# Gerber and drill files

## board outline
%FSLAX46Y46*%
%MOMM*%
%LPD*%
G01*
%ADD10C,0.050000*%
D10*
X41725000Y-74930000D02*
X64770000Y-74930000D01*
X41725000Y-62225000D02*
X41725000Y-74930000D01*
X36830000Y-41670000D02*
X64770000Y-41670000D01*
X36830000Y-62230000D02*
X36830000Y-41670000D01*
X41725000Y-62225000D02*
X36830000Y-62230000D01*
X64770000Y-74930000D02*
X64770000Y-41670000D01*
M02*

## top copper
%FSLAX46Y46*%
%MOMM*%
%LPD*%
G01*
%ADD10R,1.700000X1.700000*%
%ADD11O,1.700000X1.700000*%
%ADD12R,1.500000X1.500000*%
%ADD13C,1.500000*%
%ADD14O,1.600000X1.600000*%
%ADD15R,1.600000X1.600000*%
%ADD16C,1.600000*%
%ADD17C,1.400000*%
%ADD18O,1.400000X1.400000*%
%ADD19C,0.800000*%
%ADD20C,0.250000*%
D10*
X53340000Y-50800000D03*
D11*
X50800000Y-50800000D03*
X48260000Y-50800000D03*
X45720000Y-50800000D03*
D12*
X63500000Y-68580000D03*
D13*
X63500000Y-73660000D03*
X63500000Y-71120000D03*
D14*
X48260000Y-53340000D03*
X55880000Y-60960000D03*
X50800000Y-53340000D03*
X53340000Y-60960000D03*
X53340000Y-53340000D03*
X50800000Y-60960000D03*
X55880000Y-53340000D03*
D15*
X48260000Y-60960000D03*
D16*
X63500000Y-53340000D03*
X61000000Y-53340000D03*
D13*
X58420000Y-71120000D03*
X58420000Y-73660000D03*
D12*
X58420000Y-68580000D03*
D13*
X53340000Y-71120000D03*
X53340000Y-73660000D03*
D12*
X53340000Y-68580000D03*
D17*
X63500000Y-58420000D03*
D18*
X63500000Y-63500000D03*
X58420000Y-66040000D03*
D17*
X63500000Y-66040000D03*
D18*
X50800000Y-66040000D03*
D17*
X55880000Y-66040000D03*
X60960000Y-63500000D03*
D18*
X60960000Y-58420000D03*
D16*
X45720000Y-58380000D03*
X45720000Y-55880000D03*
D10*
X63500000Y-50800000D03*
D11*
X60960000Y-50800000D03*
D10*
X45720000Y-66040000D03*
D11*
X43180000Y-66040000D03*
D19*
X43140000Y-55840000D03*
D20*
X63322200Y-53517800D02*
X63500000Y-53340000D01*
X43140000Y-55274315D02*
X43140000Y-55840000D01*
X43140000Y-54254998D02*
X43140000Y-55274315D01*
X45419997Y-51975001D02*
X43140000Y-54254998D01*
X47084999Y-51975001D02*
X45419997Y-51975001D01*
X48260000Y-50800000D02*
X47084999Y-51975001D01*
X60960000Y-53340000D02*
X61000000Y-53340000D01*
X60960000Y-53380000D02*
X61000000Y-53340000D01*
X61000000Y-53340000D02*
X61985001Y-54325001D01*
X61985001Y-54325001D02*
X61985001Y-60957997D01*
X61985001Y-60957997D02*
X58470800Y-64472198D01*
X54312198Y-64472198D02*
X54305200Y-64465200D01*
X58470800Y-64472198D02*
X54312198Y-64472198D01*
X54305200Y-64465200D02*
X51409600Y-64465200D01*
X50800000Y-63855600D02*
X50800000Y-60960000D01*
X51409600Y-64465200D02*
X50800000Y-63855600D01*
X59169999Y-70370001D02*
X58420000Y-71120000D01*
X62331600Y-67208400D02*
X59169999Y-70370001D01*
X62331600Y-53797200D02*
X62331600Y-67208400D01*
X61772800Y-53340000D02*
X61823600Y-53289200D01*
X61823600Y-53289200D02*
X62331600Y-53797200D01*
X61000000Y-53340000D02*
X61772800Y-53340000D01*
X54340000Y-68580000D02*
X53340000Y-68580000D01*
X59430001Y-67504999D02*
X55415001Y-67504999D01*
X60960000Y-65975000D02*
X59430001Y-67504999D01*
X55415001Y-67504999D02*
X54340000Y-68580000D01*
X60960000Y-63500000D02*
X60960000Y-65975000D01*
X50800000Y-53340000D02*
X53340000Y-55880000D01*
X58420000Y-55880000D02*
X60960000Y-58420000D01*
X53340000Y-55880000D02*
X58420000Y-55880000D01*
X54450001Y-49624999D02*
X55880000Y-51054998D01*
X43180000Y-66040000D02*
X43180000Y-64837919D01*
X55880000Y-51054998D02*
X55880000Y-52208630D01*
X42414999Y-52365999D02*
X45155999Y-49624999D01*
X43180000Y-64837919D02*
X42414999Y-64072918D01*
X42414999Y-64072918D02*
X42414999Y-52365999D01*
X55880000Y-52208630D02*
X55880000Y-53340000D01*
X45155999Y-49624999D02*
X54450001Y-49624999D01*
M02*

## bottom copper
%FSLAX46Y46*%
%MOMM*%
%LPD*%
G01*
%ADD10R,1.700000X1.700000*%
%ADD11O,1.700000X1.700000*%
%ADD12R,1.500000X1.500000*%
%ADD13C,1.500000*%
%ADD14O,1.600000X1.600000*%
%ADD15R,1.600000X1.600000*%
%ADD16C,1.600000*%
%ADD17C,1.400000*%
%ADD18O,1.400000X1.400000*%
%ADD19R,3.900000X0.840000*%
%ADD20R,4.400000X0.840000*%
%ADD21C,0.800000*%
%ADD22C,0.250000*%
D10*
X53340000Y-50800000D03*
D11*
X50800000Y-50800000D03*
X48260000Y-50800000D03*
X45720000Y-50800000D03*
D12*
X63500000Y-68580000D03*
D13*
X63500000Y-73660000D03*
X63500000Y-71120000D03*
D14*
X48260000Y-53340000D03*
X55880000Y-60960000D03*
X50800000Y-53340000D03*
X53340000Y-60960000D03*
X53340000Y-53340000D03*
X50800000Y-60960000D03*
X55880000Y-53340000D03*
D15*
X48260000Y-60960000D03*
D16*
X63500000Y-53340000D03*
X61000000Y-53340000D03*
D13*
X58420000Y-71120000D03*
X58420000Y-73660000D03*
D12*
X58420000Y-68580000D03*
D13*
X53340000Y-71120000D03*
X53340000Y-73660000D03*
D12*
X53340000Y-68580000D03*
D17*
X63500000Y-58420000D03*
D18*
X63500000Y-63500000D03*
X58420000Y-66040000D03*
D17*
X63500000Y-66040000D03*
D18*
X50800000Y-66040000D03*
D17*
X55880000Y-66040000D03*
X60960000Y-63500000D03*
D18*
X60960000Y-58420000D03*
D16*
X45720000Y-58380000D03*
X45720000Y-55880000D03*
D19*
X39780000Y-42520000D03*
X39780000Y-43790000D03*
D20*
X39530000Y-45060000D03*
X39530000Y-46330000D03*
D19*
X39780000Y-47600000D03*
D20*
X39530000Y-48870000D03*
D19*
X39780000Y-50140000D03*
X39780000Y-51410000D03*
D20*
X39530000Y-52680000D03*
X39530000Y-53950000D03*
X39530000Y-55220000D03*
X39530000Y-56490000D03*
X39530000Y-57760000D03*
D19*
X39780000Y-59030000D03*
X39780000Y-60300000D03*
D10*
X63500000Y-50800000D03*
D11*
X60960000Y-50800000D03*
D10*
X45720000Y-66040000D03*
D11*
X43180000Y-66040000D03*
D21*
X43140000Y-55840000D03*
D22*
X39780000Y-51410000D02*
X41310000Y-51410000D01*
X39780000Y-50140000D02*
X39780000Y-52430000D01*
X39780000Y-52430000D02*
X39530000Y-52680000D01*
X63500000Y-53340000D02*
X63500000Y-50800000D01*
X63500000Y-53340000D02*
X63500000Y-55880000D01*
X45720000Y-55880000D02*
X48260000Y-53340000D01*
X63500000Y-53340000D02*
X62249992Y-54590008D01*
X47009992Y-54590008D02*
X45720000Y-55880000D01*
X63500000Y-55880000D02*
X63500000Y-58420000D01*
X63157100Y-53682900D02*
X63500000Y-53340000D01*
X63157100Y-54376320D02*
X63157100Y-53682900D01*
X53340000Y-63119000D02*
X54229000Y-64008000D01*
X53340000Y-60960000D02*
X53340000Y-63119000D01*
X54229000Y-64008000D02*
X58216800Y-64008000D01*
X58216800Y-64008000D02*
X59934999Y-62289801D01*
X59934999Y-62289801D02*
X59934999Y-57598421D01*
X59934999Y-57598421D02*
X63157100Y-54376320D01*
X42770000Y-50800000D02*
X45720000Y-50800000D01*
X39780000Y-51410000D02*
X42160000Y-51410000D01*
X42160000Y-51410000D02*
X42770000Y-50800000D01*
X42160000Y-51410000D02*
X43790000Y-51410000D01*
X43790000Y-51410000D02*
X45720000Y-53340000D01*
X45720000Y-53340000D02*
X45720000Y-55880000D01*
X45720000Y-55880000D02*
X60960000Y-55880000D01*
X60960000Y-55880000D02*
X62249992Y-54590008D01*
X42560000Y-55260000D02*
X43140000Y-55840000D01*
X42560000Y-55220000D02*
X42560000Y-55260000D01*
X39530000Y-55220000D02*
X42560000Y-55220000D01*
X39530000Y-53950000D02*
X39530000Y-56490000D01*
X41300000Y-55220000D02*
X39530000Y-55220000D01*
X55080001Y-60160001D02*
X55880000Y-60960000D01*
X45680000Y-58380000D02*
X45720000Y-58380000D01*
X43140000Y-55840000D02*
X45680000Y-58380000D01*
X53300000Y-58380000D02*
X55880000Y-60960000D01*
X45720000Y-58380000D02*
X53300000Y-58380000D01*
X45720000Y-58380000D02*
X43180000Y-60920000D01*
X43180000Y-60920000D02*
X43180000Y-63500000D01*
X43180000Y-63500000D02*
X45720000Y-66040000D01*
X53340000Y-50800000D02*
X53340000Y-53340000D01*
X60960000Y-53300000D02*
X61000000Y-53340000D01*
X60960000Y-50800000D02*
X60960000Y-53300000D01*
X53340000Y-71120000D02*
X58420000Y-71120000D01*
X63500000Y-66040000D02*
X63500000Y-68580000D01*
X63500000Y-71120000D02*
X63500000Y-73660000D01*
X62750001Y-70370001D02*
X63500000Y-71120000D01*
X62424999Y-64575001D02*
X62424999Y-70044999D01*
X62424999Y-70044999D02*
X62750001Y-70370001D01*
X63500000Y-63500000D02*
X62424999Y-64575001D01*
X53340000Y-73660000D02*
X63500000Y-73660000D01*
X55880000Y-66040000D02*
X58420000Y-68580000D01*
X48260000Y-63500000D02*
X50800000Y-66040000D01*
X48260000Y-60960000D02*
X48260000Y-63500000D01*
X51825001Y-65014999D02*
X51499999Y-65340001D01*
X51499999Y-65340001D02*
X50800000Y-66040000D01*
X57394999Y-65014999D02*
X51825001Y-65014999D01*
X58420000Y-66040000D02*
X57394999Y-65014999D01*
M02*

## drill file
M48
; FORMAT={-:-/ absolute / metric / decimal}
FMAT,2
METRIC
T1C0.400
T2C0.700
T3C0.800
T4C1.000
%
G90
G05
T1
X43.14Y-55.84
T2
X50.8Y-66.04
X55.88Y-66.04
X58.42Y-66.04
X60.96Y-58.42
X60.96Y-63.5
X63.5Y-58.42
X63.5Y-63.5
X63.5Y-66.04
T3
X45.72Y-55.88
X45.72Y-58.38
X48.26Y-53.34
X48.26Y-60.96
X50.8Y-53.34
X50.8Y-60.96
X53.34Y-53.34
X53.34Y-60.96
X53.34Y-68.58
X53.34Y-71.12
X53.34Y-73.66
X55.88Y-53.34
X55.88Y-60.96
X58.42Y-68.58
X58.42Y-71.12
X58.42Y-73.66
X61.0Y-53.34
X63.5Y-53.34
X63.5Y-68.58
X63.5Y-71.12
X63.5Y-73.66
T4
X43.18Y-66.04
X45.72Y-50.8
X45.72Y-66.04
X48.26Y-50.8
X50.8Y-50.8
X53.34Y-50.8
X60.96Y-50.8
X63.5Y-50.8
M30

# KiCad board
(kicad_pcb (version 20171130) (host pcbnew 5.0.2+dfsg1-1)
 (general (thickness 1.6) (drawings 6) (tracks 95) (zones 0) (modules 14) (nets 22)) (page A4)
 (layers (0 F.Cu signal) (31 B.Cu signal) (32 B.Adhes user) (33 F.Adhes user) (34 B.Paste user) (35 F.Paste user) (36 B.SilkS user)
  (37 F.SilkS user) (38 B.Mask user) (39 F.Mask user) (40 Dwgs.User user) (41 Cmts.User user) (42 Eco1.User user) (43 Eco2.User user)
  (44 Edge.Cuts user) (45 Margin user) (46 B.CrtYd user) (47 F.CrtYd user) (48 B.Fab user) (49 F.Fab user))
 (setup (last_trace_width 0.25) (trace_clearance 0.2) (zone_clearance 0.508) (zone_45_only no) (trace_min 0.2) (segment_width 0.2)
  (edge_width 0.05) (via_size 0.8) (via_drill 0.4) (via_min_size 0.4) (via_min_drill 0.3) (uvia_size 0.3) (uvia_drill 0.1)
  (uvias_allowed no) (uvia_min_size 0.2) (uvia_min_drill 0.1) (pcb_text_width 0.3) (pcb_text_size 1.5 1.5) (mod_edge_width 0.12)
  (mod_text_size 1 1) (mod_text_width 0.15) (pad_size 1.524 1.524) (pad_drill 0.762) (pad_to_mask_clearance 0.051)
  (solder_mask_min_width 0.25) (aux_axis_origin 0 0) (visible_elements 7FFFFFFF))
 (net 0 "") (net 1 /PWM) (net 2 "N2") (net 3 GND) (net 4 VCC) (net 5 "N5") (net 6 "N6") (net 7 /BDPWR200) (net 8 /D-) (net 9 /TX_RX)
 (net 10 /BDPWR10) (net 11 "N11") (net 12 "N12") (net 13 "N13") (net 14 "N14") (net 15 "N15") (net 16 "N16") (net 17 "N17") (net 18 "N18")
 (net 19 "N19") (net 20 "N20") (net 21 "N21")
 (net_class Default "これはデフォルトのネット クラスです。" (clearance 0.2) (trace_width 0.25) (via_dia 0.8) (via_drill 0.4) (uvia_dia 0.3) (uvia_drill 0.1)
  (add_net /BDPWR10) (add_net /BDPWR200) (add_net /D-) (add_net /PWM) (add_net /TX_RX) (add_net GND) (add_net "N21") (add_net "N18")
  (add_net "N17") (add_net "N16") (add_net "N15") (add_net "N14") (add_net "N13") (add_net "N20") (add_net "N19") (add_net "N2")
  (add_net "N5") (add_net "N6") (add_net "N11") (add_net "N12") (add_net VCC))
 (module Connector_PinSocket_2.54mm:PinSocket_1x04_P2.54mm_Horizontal (layer F.Cu) (at 53.34 50.8 270)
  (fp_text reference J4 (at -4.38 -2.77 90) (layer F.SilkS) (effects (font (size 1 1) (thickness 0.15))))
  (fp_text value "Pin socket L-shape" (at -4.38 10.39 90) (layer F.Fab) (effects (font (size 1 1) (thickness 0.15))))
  (pad 1 thru_hole rect (at 0 0 270) (size 1.7 1.7) (drill 1) (layers *.Cu *.Mask) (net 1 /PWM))
  (pad 2 thru_hole oval (at 0 2.54 270) (size 1.7 1.7) (drill 1) (layers *.Cu *.Mask) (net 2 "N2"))
  (pad 3 thru_hole oval (at 0 5.08 270) (size 1.7 1.7) (drill 1) (layers *.Cu *.Mask) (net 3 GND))
  (pad 4 thru_hole oval (at 0 7.62 270) (size 1.7 1.7) (drill 1) (layers *.Cu *.Mask) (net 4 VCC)))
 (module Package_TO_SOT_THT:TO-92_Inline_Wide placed (layer F.Cu) (at 63.5 68.58 270)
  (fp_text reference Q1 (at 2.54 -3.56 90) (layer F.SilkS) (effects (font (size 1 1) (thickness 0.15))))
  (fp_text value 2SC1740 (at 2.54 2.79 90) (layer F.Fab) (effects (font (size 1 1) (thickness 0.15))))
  (pad 1 thru_hole rect (at 0 0) (size 1.5 1.5) (drill 0.8) (layers *.Cu *.Mask) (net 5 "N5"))
  (pad 3 thru_hole circle (at 5.08 0) (size 1.5 1.5) (drill 0.8) (layers *.Cu *.Mask) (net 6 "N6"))
  (pad 2 thru_hole circle (at 2.54 0) (size 1.5 1.5) (drill 0.8) (layers *.Cu *.Mask) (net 6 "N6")))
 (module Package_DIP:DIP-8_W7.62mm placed (layer F.Cu) (at 48.26 60.96 90)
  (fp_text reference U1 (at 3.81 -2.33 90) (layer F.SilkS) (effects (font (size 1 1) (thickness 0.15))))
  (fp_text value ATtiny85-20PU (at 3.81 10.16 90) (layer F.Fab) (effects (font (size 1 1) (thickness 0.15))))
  (pad 8 thru_hole oval (at 7.62 0 90) (size 1.6 1.6) (drill 0.8) (layers *.Cu *.Mask) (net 4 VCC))
  (pad 4 thru_hole oval (at 0 7.62 90) (size 1.6 1.6) (drill 0.8) (layers *.Cu *.Mask) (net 3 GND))
  (pad 7 thru_hole oval (at 7.62 2.54 90) (size 1.6 1.6) (drill 0.8) (layers *.Cu *.Mask) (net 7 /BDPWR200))
  (pad 3 thru_hole oval (at 0 5.08 90) (size 1.6 1.6) (drill 0.8) (layers *.Cu *.Mask) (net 4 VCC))
  (pad 6 thru_hole oval (at 7.62 5.08 90) (size 1.6 1.6) (drill 0.8) (layers *.Cu *.Mask) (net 1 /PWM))
  (pad 2 thru_hole oval (at 0 2.54 90) (size 1.6 1.6) (drill 0.8) (layers *.Cu *.Mask) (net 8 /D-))
  (pad 5 thru_hole oval (at 7.62 7.62 90) (size 1.6 1.6) (drill 0.8) (layers *.Cu *.Mask) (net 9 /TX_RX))
  (pad 1 thru_hole rect (at 0 0 90) (size 1.6 1.6) (drill 0.8) (layers *.Cu *.Mask) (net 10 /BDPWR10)))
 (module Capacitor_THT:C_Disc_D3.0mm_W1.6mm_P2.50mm (layer F.Cu) (at 63.5 53.34 180)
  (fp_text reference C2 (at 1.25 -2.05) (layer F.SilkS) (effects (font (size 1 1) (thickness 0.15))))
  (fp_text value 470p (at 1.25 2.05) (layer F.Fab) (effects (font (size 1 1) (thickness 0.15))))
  (pad 1 thru_hole circle (at 0 0 180) (size 1.6 1.6) (drill 0.8) (layers *.Cu *.Mask) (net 4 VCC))
  (pad 2 thru_hole circle (at 2.5 0 180) (size 1.6 1.6) (drill 0.8) (layers *.Cu *.Mask) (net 8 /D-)))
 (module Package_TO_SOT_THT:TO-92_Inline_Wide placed (layer F.Cu) (at 58.42 68.58 270)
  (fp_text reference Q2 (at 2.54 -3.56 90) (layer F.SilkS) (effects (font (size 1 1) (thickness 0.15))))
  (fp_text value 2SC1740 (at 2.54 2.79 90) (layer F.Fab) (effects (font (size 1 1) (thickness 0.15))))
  (pad 2 thru_hole circle (at 2.54 0) (size 1.5 1.5) (drill 0.8) (layers *.Cu *.Mask) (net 8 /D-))
  (pad 3 thru_hole circle (at 5.08 0) (size 1.5 1.5) (drill 0.8) (layers *.Cu *.Mask) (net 6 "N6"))
  (pad 1 thru_hole rect (at 0 0) (size 1.5 1.5) (drill 0.8) (layers *.Cu *.Mask) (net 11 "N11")))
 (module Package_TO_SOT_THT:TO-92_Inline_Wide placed (layer F.Cu) (at 53.34 68.58 270)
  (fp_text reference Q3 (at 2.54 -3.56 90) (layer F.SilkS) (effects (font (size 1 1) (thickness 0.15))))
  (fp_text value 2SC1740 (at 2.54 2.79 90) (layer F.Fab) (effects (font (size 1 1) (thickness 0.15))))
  (pad 2 thru_hole circle (at 2.54 0) (size 1.5 1.5) (drill 0.8) (layers *.Cu *.Mask) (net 8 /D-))
  (pad 3 thru_hole circle (at 5.08 0) (size 1.5 1.5) (drill 0.8) (layers *.Cu *.Mask) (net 6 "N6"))
  (pad 1 thru_hole rect (at 0 0) (size 1.5 1.5) (drill 0.8) (layers *.Cu *.Mask) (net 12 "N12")))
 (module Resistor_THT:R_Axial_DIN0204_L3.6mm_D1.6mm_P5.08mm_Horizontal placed (layer F.Cu) (at 63.5 58.42 270)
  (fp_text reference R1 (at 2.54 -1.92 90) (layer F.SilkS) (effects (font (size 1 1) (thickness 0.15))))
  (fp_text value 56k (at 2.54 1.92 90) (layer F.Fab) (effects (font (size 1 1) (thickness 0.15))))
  (pad 1 thru_hole circle (at 0 0 270) (size 1.4 1.4) (drill 0.7) (layers *.Cu *.Mask) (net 4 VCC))
  (pad 2 thru_hole oval (at 5.08 0 270) (size 1.4 1.4) (drill 0.7) (layers *.Cu *.Mask) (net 6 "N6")))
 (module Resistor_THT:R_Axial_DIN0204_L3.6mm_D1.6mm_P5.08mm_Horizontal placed (layer F.Cu) (at 63.5 66.04 180)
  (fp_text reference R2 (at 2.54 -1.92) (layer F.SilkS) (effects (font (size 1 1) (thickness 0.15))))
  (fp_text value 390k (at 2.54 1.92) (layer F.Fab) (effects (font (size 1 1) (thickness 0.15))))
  (pad 2 thru_hole oval (at 5.08 0 180) (size 1.4 1.4) (drill 0.7) (layers *.Cu *.Mask) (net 10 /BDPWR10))
  (pad 1 thru_hole circle (at 0 0 180) (size 1.4 1.4) (drill 0.7) (layers *.Cu *.Mask) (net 5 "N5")))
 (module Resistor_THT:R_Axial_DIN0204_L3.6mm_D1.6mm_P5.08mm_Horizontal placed (layer F.Cu) (at 55.88 66.04 180)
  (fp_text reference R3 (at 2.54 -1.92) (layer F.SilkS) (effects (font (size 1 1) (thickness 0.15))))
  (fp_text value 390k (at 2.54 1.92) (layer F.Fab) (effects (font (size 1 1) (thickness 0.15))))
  (pad 2 thru_hole oval (at 5.08 0 180) (size 1.4 1.4) (drill 0.7) (layers *.Cu *.Mask) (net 10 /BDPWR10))
  (pad 1 thru_hole circle (at 0 0 180) (size 1.4 1.4) (drill 0.7) (layers *.Cu *.Mask) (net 11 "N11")))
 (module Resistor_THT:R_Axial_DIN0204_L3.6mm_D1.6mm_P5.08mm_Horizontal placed (layer F.Cu) (at 60.96 63.5 90)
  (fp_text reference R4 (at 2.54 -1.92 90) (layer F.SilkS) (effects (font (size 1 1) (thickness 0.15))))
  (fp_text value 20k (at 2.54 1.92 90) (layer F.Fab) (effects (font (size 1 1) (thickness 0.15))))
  (pad 1 thru_hole circle (at 0 0 90) (size 1.4 1.4) (drill 0.7) (layers *.Cu *.Mask) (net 12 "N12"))
  (pad 2 thru_hole oval (at 5.08 0 90) (size 1.4 1.4) (drill 0.7) (layers *.Cu *.Mask) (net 7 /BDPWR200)))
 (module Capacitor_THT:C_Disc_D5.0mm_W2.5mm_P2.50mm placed (layer F.Cu) (at 45.72 55.88 270)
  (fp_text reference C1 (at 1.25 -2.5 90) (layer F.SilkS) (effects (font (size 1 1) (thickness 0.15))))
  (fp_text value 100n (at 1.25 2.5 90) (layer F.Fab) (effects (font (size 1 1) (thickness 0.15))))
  (pad 2 thru_hole circle (at 2.5 0 270) (size 1.6 1.6) (drill 0.8) (layers *.Cu *.Mask) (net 3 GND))
  (pad 1 thru_hole circle (at 0 0 270) (size 1.6 1.6) (drill 0.8) (layers *.Cu *.Mask) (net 4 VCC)))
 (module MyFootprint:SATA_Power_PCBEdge (layer B.Cu) (at 41.73 60.72 270)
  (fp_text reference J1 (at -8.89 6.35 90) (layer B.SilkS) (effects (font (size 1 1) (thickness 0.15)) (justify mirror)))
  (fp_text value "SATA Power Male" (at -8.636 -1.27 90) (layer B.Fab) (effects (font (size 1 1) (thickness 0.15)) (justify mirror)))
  (pad 15 smd rect (at -18.2 1.95 270) (size 0.84 3.9) (layers B.Cu B.Paste B.Mask) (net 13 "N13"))
  (pad 14 smd rect (at -16.93 1.95 270) (size 0.84 3.9) (layers B.Cu B.Paste B.Mask) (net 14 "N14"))
  (pad 13 smd rect (at -15.66 2.2 270) (size 0.84 4.4) (layers B.Cu B.Paste B.Mask) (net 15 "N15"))
  (pad 12 smd rect (at -14.39 2.2 270) (size 0.84 4.4) (layers B.Cu B.Paste B.Mask) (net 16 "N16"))
  (pad 11 smd rect (at -13.12 1.95 270) (size 0.84 3.9) (layers B.Cu B.Paste B.Mask) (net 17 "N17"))
  (pad 10 smd rect (at -11.85 2.2 270) (size 0.84 4.4) (layers B.Cu B.Paste B.Mask) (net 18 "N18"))
  (pad 9 smd rect (at -10.58 1.95 270) (size 0.84 3.9) (layers B.Cu B.Paste B.Mask) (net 4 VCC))
  (pad 8 smd rect (at -9.31 1.95 270) (size 0.84 3.9) (layers B.Cu B.Paste B.Mask) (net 4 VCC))
  (pad 7 smd rect (at -8.04 2.2 270) (size 0.84 4.4) (layers B.Cu B.Paste B.Mask) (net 4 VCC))
  (pad 6 smd rect (at -6.77 2.2 270) (size 0.84 4.4) (layers B.Cu B.Paste B.Mask) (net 3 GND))
  (pad 5 smd rect (at -5.5 2.2 270) (size 0.84 4.4) (layers B.Cu B.Paste B.Mask) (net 3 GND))
  (pad 4 smd rect (at -4.23 2.2 270) (size 0.84 4.4) (layers B.Cu B.Paste B.Mask) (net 3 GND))
  (pad 3 smd rect (at -2.96 2.2 270) (size 0.84 4.4) (layers B.Cu B.Paste B.Mask) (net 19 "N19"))
  (pad 2 smd rect (at -1.69 1.95 270) (size 0.84 3.9) (layers B.Cu B.Paste B.Mask) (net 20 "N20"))
  (pad 1 smd rect (at -0.42 1.95 270) (size 0.84 3.9) (layers B.Cu B.Paste B.Mask) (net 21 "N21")))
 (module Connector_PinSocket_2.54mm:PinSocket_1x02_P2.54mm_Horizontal (layer F.Cu) (at 63.5 50.8 270)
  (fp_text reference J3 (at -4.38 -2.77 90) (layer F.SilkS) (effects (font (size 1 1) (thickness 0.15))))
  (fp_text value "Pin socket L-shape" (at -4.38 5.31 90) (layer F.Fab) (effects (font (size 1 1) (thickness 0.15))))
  (pad 1 thru_hole rect (at 0 0 270) (size 1.7 1.7) (drill 1) (layers *.Cu *.Mask) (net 4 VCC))
  (pad 2 thru_hole oval (at 0 2.54 270) (size 1.7 1.7) (drill 1) (layers *.Cu *.Mask) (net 8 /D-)))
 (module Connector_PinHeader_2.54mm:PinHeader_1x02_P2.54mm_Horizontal (layer F.Cu) (at 45.72 66.04 270)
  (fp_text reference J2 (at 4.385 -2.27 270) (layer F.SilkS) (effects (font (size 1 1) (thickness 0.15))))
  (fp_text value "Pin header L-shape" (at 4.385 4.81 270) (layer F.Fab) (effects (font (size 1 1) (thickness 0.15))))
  (pad 1 thru_hole rect (at 0 0 270) (size 1.7 1.7) (drill 1) (layers *.Cu *.Mask) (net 3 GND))
  (pad 2 thru_hole oval (at 0 2.54 270) (size 1.7 1.7) (drill 1) (layers *.Cu *.Mask) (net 9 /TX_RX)))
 (gr_line (start 41.725 74.93) (end 64.77 74.93) (layer Edge.Cuts) (width 0.05))
 (gr_line (start 41.725 62.225) (end 41.725 74.93) (layer Edge.Cuts) (width 0.05))
 (gr_line (start 36.83 41.67) (end 64.77 41.67) (layer Edge.Cuts) (width 0.05))
 (gr_line (start 36.83 62.23) (end 36.83 41.67) (layer Edge.Cuts) (width 0.05))
 (gr_line (start 41.725 62.225) (end 36.83 62.23) (layer Edge.Cuts) (width 0.05))
 (gr_line (start 64.77 74.93) (end 64.77 41.67) (layer Edge.Cuts) (width 0.05))
 (segment (start 39.78 51.41) (end 41.31 51.41) (width 0.25) (layer B.Cu) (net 4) (status 30))
 (segment (start 39.78 50.14) (end 39.78 52.43) (width 0.25) (layer B.Cu) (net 4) (status 30))
 (segment (start 39.78 52.43) (end 39.53 52.68) (width 0.25) (layer B.Cu) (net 4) (status 30))
 (segment (start 63.5 53.34) (end 63.5 50.8) (width 0.25) (layer B.Cu) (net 4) (status 30))
 (segment (start 63.5 53.34) (end 63.5 55.88) (width 0.25) (layer B.Cu) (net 4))
 (segment (start 63.3222 53.5178) (end 63.5 53.34) (width 0.25) (layer F.Cu) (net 4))
 (segment (start 45.72 55.88) (end 48.26 53.34) (width 0.25) (layer B.Cu) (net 4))
 (segment (start 63.5 53.34) (end 62.249992 54.590008) (width 0.25) (layer B.Cu) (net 4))
 (segment (start 47.009992 54.590008) (end 45.72 55.88) (width 0.25) (layer B.Cu) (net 4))
 (segment (start 63.5 55.88) (end 63.5 58.42) (width 0.25) (layer B.Cu) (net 4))
 (segment (start 63.1571 53.6829) (end 63.5 53.34) (width 0.25) (layer B.Cu) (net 4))
 (segment (start 63.1571 54.37632) (end 63.1571 53.6829) (width 0.25) (layer B.Cu) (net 4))
 (segment (start 53.34 63.119) (end 54.229 64.008) (width 0.25) (layer B.Cu) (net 4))
 (segment (start 53.34 60.96) (end 53.34 63.119) (width 0.25) (layer B.Cu) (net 4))
 (segment (start 54.229 64.008) (end 58.2168 64.008) (width 0.25) (layer B.Cu) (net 4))
 (segment (start 58.2168 64.008) (end 59.934999 62.289801) (width 0.25) (layer B.Cu) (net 4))
 (segment (start 59.934999 62.289801) (end 59.934999 57.598421) (width 0.25) (layer B.Cu) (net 4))
 (segment (start 59.934999 57.598421) (end 63.1571 54.37632) (width 0.25) (layer B.Cu) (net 4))
 (segment (start 42.77 50.8) (end 45.72 50.8) (width 0.25) (layer B.Cu) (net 4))
 (segment (start 39.78 51.41) (end 42.16 51.41) (width 0.25) (layer B.Cu) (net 4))
 (segment (start 42.16 51.41) (end 42.77 50.8) (width 0.25) (layer B.Cu) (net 4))
 (segment (start 42.16 51.41) (end 43.79 51.41) (width 0.25) (layer B.Cu) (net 4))
 (segment (start 43.79 51.41) (end 45.72 53.34) (width 0.25) (layer B.Cu) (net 4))
 (segment (start 45.72 53.34) (end 45.72 55.88) (width 0.25) (layer B.Cu) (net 4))
 (segment (start 45.72 55.88) (end 60.96 55.88) (width 0.25) (layer B.Cu) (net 4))
 (segment (start 60.96 55.88) (end 62.249992 54.590008) (width 0.25) (layer B.Cu) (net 4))
 (segment (start 42.56 55.26) (end 43.14 55.84) (width 0.25) (layer B.Cu) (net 3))
 (segment (start 42.56 55.22) (end 42.56 55.26) (width 0.25) (layer B.Cu) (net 3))
 (segment (start 39.53 55.22) (end 42.56 55.22) (width 0.25) (layer B.Cu) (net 3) (status 10))
 (segment (start 39.53 53.95) (end 39.53 56.49) (width 0.25) (layer B.Cu) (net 3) (status 30))
 (segment (start 41.3 55.22) (end 39.53 55.22) (width 0.25) (layer B.Cu) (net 3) (status 30))
 (via (at 43.14 55.84) (size 0.8) (drill 0.4) (layers F.Cu B.Cu) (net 3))
 (segment (start 43.14 55.274315) (end 43.14 55.84) (width 0.25) (layer F.Cu) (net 3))
 (segment (start 43.14 54.254998) (end 43.14 55.274315) (width 0.25) (layer F.Cu) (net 3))
 (segment (start 45.419997 51.975001) (end 43.14 54.254998) (width 0.25) (layer F.Cu) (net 3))
 (segment (start 47.084999 51.975001) (end 45.419997 51.975001) (width 0.25) (layer F.Cu) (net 3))
 (segment (start 48.26 50.8) (end 47.084999 51.975001) (width 0.25) (layer F.Cu) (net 3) (status 10))
 (segment (start 55.080001 60.160001) (end 55.88 60.96) (width 0.25) (layer B.Cu) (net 3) (status 20))
 (segment (start 45.68 58.38) (end 45.72 58.38) (width 0.25) (layer B.Cu) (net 3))
 (segment (start 43.14 55.84) (end 45.68 58.38) (width 0.25) (layer B.Cu) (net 3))
 (segment (start 53.3 58.38) (end 55.88 60.96) (width 0.25) (layer B.Cu) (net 3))
 (segment (start 45.72 58.38) (end 53.3 58.38) (width 0.25) (layer B.Cu) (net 3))
 (segment (start 45.72 58.38) (end 43.18 60.92) (width 0.25) (layer B.Cu) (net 3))
 (segment (start 43.18 60.92) (end 43.18 63.5) (width 0.25) (layer B.Cu) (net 3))
 (segment (start 43.18 63.5) (end 45.72 66.04) (width 0.25) (layer B.Cu) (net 3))
 (segment (start 53.34 50.8) (end 53.34 53.34) (width 0.25) (layer B.Cu) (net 1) (status 30))
 (segment (start 60.96 53.34) (end 61 53.34) (width 0.25) (layer F.Cu) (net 8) (status 30))
 (segment (start 60.96 53.3) (end 61 53.34) (width 0.25) (layer B.Cu) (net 8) (status 30))
 (segment (start 60.96 53.38) (end 61 53.34) (width 0.25) (layer F.Cu) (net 8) (status 30))
 (segment (start 60.96 50.8) (end 60.96 53.3) (width 0.25) (layer B.Cu) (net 8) (status 30))
 (segment (start 53.34 71.12) (end 58.42 71.12) (width 0.25) (layer B.Cu) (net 8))
 (segment (start 61 53.34) (end 61.985001 54.325001) (width 0.25) (layer F.Cu) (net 8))
 (segment (start 61.985001 54.325001) (end 61.985001 60.957997) (width 0.25) (layer F.Cu) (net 8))
 (segment (start 61.985001 60.957997) (end 58.4708 64.472198) (width 0.25) (layer F.Cu) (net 8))
 (segment (start 54.312198 64.472198) (end 54.3052 64.4652) (width 0.25) (layer F.Cu) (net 8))
 (segment (start 58.4708 64.472198) (end 54.312198 64.472198) (width 0.25) (layer F.Cu) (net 8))
 (segment (start 54.3052 64.4652) (end 51.4096 64.4652) (width 0.25) (layer F.Cu) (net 8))
 (segment (start 50.8 63.8556) (end 50.8 60.96) (width 0.25) (layer F.Cu) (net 8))
 (segment (start 51.4096 64.4652) (end 50.8 63.8556) (width 0.25) (layer F.Cu) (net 8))
 (segment (start 59.169999 70.370001) (end 58.42 71.12) (width 0.25) (layer F.Cu) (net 8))
 (segment (start 62.3316 67.2084) (end 59.169999 70.370001) (width 0.25) (layer F.Cu) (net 8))
 (segment (start 62.3316 53.7972) (end 62.3316 67.2084) (width 0.25) (layer F.Cu) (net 8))
 (segment (start 61.7728 53.34) (end 61.8236 53.2892) (width 0.25) (layer F.Cu) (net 8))
 (segment (start 61.8236 53.2892) (end 62.3316 53.7972) (width 0.25) (layer F.Cu) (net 8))
 (segment (start 61 53.34) (end 61.7728 53.34) (width 0.25) (layer F.Cu) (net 8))
 (segment (start 63.5 66.04) (end 63.5 68.58) (width 0.25) (layer B.Cu) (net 5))
 (segment (start 63.5 71.12) (end 63.5 73.66) (width 0.25) (layer B.Cu) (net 6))
 (segment (start 62.750001 70.370001) (end 63.5 71.12) (width 0.25) (layer B.Cu) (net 6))
 (segment (start 62.424999 64.575001) (end 62.424999 70.044999) (width 0.25) (layer B.Cu) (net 6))
 (segment (start 62.424999 70.044999) (end 62.750001 70.370001) (width 0.25) (layer B.Cu) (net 6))
 (segment (start 63.5 63.5) (end 62.424999 64.575001) (width 0.25) (layer B.Cu) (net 6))
 (segment (start 53.34 73.66) (end 63.5 73.66) (width 0.25) (layer B.Cu) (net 6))
 (segment (start 55.88 66.04) (end 58.42 68.58) (width 0.25) (layer B.Cu) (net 11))
 (segment (start 54.34 68.58) (end 53.34 68.58) (width 0.25) (layer F.Cu) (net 12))
 (segment (start 59.430001 67.504999) (end 55.415001 67.504999) (width 0.25) (layer F.Cu) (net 12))
 (segment (start 60.96 65.975) (end 59.430001 67.504999) (width 0.25) (layer F.Cu) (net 12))
 (segment (start 55.415001 67.504999) (end 54.34 68.58) (width 0.25) (layer F.Cu) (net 12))
 (segment (start 60.96 63.5) (end 60.96 65.975) (width 0.25) (layer F.Cu) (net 12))
 (segment (start 48.26 63.5) (end 50.8 66.04) (width 0.25) (layer B.Cu) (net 10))
 (segment (start 48.26 60.96) (end 48.26 63.5) (width 0.25) (layer B.Cu) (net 10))
 (segment (start 51.825001 65.014999) (end 51.499999 65.340001) (width 0.25) (layer B.Cu) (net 10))
 (segment (start 51.499999 65.340001) (end 50.8 66.04) (width 0.25) (layer B.Cu) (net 10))
 (segment (start 57.394999 65.014999) (end 51.825001 65.014999) (width 0.25) (layer B.Cu) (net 10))
 (segment (start 58.42 66.04) (end 57.394999 65.014999) (width 0.25) (layer B.Cu) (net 10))
 (segment (start 50.8 53.34) (end 53.34 55.88) (width 0.25) (layer F.Cu) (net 7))
 (segment (start 58.42 55.88) (end 60.96 58.42) (width 0.25) (layer F.Cu) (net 7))
 (segment (start 53.34 55.88) (end 58.42 55.88) (width 0.25) (layer F.Cu) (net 7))
 (segment (start 54.450001 49.624999) (end 55.88 51.054998) (width 0.25) (layer F.Cu) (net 9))
 (segment (start 43.18 66.04) (end 43.18 64.837919) (width 0.25) (layer F.Cu) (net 9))
 (segment (start 55.88 51.054998) (end 55.88 52.20863) (width 0.25) (layer F.Cu) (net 9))
 (segment (start 42.414999 52.365999) (end 45.155999 49.624999) (width 0.25) (layer F.Cu) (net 9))
 (segment (start 43.18 64.837919) (end 42.414999 64.072918) (width 0.25) (layer F.Cu) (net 9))
 (segment (start 42.414999 64.072918) (end 42.414999 52.365999) (width 0.25) (layer F.Cu) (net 9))
 (segment (start 55.88 52.20863) (end 55.88 53.34) (width 0.25) (layer F.Cu) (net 9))
 (segment (start 45.155999 49.624999) (end 54.450001 49.624999) (width 0.25) (layer F.Cu) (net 9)))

